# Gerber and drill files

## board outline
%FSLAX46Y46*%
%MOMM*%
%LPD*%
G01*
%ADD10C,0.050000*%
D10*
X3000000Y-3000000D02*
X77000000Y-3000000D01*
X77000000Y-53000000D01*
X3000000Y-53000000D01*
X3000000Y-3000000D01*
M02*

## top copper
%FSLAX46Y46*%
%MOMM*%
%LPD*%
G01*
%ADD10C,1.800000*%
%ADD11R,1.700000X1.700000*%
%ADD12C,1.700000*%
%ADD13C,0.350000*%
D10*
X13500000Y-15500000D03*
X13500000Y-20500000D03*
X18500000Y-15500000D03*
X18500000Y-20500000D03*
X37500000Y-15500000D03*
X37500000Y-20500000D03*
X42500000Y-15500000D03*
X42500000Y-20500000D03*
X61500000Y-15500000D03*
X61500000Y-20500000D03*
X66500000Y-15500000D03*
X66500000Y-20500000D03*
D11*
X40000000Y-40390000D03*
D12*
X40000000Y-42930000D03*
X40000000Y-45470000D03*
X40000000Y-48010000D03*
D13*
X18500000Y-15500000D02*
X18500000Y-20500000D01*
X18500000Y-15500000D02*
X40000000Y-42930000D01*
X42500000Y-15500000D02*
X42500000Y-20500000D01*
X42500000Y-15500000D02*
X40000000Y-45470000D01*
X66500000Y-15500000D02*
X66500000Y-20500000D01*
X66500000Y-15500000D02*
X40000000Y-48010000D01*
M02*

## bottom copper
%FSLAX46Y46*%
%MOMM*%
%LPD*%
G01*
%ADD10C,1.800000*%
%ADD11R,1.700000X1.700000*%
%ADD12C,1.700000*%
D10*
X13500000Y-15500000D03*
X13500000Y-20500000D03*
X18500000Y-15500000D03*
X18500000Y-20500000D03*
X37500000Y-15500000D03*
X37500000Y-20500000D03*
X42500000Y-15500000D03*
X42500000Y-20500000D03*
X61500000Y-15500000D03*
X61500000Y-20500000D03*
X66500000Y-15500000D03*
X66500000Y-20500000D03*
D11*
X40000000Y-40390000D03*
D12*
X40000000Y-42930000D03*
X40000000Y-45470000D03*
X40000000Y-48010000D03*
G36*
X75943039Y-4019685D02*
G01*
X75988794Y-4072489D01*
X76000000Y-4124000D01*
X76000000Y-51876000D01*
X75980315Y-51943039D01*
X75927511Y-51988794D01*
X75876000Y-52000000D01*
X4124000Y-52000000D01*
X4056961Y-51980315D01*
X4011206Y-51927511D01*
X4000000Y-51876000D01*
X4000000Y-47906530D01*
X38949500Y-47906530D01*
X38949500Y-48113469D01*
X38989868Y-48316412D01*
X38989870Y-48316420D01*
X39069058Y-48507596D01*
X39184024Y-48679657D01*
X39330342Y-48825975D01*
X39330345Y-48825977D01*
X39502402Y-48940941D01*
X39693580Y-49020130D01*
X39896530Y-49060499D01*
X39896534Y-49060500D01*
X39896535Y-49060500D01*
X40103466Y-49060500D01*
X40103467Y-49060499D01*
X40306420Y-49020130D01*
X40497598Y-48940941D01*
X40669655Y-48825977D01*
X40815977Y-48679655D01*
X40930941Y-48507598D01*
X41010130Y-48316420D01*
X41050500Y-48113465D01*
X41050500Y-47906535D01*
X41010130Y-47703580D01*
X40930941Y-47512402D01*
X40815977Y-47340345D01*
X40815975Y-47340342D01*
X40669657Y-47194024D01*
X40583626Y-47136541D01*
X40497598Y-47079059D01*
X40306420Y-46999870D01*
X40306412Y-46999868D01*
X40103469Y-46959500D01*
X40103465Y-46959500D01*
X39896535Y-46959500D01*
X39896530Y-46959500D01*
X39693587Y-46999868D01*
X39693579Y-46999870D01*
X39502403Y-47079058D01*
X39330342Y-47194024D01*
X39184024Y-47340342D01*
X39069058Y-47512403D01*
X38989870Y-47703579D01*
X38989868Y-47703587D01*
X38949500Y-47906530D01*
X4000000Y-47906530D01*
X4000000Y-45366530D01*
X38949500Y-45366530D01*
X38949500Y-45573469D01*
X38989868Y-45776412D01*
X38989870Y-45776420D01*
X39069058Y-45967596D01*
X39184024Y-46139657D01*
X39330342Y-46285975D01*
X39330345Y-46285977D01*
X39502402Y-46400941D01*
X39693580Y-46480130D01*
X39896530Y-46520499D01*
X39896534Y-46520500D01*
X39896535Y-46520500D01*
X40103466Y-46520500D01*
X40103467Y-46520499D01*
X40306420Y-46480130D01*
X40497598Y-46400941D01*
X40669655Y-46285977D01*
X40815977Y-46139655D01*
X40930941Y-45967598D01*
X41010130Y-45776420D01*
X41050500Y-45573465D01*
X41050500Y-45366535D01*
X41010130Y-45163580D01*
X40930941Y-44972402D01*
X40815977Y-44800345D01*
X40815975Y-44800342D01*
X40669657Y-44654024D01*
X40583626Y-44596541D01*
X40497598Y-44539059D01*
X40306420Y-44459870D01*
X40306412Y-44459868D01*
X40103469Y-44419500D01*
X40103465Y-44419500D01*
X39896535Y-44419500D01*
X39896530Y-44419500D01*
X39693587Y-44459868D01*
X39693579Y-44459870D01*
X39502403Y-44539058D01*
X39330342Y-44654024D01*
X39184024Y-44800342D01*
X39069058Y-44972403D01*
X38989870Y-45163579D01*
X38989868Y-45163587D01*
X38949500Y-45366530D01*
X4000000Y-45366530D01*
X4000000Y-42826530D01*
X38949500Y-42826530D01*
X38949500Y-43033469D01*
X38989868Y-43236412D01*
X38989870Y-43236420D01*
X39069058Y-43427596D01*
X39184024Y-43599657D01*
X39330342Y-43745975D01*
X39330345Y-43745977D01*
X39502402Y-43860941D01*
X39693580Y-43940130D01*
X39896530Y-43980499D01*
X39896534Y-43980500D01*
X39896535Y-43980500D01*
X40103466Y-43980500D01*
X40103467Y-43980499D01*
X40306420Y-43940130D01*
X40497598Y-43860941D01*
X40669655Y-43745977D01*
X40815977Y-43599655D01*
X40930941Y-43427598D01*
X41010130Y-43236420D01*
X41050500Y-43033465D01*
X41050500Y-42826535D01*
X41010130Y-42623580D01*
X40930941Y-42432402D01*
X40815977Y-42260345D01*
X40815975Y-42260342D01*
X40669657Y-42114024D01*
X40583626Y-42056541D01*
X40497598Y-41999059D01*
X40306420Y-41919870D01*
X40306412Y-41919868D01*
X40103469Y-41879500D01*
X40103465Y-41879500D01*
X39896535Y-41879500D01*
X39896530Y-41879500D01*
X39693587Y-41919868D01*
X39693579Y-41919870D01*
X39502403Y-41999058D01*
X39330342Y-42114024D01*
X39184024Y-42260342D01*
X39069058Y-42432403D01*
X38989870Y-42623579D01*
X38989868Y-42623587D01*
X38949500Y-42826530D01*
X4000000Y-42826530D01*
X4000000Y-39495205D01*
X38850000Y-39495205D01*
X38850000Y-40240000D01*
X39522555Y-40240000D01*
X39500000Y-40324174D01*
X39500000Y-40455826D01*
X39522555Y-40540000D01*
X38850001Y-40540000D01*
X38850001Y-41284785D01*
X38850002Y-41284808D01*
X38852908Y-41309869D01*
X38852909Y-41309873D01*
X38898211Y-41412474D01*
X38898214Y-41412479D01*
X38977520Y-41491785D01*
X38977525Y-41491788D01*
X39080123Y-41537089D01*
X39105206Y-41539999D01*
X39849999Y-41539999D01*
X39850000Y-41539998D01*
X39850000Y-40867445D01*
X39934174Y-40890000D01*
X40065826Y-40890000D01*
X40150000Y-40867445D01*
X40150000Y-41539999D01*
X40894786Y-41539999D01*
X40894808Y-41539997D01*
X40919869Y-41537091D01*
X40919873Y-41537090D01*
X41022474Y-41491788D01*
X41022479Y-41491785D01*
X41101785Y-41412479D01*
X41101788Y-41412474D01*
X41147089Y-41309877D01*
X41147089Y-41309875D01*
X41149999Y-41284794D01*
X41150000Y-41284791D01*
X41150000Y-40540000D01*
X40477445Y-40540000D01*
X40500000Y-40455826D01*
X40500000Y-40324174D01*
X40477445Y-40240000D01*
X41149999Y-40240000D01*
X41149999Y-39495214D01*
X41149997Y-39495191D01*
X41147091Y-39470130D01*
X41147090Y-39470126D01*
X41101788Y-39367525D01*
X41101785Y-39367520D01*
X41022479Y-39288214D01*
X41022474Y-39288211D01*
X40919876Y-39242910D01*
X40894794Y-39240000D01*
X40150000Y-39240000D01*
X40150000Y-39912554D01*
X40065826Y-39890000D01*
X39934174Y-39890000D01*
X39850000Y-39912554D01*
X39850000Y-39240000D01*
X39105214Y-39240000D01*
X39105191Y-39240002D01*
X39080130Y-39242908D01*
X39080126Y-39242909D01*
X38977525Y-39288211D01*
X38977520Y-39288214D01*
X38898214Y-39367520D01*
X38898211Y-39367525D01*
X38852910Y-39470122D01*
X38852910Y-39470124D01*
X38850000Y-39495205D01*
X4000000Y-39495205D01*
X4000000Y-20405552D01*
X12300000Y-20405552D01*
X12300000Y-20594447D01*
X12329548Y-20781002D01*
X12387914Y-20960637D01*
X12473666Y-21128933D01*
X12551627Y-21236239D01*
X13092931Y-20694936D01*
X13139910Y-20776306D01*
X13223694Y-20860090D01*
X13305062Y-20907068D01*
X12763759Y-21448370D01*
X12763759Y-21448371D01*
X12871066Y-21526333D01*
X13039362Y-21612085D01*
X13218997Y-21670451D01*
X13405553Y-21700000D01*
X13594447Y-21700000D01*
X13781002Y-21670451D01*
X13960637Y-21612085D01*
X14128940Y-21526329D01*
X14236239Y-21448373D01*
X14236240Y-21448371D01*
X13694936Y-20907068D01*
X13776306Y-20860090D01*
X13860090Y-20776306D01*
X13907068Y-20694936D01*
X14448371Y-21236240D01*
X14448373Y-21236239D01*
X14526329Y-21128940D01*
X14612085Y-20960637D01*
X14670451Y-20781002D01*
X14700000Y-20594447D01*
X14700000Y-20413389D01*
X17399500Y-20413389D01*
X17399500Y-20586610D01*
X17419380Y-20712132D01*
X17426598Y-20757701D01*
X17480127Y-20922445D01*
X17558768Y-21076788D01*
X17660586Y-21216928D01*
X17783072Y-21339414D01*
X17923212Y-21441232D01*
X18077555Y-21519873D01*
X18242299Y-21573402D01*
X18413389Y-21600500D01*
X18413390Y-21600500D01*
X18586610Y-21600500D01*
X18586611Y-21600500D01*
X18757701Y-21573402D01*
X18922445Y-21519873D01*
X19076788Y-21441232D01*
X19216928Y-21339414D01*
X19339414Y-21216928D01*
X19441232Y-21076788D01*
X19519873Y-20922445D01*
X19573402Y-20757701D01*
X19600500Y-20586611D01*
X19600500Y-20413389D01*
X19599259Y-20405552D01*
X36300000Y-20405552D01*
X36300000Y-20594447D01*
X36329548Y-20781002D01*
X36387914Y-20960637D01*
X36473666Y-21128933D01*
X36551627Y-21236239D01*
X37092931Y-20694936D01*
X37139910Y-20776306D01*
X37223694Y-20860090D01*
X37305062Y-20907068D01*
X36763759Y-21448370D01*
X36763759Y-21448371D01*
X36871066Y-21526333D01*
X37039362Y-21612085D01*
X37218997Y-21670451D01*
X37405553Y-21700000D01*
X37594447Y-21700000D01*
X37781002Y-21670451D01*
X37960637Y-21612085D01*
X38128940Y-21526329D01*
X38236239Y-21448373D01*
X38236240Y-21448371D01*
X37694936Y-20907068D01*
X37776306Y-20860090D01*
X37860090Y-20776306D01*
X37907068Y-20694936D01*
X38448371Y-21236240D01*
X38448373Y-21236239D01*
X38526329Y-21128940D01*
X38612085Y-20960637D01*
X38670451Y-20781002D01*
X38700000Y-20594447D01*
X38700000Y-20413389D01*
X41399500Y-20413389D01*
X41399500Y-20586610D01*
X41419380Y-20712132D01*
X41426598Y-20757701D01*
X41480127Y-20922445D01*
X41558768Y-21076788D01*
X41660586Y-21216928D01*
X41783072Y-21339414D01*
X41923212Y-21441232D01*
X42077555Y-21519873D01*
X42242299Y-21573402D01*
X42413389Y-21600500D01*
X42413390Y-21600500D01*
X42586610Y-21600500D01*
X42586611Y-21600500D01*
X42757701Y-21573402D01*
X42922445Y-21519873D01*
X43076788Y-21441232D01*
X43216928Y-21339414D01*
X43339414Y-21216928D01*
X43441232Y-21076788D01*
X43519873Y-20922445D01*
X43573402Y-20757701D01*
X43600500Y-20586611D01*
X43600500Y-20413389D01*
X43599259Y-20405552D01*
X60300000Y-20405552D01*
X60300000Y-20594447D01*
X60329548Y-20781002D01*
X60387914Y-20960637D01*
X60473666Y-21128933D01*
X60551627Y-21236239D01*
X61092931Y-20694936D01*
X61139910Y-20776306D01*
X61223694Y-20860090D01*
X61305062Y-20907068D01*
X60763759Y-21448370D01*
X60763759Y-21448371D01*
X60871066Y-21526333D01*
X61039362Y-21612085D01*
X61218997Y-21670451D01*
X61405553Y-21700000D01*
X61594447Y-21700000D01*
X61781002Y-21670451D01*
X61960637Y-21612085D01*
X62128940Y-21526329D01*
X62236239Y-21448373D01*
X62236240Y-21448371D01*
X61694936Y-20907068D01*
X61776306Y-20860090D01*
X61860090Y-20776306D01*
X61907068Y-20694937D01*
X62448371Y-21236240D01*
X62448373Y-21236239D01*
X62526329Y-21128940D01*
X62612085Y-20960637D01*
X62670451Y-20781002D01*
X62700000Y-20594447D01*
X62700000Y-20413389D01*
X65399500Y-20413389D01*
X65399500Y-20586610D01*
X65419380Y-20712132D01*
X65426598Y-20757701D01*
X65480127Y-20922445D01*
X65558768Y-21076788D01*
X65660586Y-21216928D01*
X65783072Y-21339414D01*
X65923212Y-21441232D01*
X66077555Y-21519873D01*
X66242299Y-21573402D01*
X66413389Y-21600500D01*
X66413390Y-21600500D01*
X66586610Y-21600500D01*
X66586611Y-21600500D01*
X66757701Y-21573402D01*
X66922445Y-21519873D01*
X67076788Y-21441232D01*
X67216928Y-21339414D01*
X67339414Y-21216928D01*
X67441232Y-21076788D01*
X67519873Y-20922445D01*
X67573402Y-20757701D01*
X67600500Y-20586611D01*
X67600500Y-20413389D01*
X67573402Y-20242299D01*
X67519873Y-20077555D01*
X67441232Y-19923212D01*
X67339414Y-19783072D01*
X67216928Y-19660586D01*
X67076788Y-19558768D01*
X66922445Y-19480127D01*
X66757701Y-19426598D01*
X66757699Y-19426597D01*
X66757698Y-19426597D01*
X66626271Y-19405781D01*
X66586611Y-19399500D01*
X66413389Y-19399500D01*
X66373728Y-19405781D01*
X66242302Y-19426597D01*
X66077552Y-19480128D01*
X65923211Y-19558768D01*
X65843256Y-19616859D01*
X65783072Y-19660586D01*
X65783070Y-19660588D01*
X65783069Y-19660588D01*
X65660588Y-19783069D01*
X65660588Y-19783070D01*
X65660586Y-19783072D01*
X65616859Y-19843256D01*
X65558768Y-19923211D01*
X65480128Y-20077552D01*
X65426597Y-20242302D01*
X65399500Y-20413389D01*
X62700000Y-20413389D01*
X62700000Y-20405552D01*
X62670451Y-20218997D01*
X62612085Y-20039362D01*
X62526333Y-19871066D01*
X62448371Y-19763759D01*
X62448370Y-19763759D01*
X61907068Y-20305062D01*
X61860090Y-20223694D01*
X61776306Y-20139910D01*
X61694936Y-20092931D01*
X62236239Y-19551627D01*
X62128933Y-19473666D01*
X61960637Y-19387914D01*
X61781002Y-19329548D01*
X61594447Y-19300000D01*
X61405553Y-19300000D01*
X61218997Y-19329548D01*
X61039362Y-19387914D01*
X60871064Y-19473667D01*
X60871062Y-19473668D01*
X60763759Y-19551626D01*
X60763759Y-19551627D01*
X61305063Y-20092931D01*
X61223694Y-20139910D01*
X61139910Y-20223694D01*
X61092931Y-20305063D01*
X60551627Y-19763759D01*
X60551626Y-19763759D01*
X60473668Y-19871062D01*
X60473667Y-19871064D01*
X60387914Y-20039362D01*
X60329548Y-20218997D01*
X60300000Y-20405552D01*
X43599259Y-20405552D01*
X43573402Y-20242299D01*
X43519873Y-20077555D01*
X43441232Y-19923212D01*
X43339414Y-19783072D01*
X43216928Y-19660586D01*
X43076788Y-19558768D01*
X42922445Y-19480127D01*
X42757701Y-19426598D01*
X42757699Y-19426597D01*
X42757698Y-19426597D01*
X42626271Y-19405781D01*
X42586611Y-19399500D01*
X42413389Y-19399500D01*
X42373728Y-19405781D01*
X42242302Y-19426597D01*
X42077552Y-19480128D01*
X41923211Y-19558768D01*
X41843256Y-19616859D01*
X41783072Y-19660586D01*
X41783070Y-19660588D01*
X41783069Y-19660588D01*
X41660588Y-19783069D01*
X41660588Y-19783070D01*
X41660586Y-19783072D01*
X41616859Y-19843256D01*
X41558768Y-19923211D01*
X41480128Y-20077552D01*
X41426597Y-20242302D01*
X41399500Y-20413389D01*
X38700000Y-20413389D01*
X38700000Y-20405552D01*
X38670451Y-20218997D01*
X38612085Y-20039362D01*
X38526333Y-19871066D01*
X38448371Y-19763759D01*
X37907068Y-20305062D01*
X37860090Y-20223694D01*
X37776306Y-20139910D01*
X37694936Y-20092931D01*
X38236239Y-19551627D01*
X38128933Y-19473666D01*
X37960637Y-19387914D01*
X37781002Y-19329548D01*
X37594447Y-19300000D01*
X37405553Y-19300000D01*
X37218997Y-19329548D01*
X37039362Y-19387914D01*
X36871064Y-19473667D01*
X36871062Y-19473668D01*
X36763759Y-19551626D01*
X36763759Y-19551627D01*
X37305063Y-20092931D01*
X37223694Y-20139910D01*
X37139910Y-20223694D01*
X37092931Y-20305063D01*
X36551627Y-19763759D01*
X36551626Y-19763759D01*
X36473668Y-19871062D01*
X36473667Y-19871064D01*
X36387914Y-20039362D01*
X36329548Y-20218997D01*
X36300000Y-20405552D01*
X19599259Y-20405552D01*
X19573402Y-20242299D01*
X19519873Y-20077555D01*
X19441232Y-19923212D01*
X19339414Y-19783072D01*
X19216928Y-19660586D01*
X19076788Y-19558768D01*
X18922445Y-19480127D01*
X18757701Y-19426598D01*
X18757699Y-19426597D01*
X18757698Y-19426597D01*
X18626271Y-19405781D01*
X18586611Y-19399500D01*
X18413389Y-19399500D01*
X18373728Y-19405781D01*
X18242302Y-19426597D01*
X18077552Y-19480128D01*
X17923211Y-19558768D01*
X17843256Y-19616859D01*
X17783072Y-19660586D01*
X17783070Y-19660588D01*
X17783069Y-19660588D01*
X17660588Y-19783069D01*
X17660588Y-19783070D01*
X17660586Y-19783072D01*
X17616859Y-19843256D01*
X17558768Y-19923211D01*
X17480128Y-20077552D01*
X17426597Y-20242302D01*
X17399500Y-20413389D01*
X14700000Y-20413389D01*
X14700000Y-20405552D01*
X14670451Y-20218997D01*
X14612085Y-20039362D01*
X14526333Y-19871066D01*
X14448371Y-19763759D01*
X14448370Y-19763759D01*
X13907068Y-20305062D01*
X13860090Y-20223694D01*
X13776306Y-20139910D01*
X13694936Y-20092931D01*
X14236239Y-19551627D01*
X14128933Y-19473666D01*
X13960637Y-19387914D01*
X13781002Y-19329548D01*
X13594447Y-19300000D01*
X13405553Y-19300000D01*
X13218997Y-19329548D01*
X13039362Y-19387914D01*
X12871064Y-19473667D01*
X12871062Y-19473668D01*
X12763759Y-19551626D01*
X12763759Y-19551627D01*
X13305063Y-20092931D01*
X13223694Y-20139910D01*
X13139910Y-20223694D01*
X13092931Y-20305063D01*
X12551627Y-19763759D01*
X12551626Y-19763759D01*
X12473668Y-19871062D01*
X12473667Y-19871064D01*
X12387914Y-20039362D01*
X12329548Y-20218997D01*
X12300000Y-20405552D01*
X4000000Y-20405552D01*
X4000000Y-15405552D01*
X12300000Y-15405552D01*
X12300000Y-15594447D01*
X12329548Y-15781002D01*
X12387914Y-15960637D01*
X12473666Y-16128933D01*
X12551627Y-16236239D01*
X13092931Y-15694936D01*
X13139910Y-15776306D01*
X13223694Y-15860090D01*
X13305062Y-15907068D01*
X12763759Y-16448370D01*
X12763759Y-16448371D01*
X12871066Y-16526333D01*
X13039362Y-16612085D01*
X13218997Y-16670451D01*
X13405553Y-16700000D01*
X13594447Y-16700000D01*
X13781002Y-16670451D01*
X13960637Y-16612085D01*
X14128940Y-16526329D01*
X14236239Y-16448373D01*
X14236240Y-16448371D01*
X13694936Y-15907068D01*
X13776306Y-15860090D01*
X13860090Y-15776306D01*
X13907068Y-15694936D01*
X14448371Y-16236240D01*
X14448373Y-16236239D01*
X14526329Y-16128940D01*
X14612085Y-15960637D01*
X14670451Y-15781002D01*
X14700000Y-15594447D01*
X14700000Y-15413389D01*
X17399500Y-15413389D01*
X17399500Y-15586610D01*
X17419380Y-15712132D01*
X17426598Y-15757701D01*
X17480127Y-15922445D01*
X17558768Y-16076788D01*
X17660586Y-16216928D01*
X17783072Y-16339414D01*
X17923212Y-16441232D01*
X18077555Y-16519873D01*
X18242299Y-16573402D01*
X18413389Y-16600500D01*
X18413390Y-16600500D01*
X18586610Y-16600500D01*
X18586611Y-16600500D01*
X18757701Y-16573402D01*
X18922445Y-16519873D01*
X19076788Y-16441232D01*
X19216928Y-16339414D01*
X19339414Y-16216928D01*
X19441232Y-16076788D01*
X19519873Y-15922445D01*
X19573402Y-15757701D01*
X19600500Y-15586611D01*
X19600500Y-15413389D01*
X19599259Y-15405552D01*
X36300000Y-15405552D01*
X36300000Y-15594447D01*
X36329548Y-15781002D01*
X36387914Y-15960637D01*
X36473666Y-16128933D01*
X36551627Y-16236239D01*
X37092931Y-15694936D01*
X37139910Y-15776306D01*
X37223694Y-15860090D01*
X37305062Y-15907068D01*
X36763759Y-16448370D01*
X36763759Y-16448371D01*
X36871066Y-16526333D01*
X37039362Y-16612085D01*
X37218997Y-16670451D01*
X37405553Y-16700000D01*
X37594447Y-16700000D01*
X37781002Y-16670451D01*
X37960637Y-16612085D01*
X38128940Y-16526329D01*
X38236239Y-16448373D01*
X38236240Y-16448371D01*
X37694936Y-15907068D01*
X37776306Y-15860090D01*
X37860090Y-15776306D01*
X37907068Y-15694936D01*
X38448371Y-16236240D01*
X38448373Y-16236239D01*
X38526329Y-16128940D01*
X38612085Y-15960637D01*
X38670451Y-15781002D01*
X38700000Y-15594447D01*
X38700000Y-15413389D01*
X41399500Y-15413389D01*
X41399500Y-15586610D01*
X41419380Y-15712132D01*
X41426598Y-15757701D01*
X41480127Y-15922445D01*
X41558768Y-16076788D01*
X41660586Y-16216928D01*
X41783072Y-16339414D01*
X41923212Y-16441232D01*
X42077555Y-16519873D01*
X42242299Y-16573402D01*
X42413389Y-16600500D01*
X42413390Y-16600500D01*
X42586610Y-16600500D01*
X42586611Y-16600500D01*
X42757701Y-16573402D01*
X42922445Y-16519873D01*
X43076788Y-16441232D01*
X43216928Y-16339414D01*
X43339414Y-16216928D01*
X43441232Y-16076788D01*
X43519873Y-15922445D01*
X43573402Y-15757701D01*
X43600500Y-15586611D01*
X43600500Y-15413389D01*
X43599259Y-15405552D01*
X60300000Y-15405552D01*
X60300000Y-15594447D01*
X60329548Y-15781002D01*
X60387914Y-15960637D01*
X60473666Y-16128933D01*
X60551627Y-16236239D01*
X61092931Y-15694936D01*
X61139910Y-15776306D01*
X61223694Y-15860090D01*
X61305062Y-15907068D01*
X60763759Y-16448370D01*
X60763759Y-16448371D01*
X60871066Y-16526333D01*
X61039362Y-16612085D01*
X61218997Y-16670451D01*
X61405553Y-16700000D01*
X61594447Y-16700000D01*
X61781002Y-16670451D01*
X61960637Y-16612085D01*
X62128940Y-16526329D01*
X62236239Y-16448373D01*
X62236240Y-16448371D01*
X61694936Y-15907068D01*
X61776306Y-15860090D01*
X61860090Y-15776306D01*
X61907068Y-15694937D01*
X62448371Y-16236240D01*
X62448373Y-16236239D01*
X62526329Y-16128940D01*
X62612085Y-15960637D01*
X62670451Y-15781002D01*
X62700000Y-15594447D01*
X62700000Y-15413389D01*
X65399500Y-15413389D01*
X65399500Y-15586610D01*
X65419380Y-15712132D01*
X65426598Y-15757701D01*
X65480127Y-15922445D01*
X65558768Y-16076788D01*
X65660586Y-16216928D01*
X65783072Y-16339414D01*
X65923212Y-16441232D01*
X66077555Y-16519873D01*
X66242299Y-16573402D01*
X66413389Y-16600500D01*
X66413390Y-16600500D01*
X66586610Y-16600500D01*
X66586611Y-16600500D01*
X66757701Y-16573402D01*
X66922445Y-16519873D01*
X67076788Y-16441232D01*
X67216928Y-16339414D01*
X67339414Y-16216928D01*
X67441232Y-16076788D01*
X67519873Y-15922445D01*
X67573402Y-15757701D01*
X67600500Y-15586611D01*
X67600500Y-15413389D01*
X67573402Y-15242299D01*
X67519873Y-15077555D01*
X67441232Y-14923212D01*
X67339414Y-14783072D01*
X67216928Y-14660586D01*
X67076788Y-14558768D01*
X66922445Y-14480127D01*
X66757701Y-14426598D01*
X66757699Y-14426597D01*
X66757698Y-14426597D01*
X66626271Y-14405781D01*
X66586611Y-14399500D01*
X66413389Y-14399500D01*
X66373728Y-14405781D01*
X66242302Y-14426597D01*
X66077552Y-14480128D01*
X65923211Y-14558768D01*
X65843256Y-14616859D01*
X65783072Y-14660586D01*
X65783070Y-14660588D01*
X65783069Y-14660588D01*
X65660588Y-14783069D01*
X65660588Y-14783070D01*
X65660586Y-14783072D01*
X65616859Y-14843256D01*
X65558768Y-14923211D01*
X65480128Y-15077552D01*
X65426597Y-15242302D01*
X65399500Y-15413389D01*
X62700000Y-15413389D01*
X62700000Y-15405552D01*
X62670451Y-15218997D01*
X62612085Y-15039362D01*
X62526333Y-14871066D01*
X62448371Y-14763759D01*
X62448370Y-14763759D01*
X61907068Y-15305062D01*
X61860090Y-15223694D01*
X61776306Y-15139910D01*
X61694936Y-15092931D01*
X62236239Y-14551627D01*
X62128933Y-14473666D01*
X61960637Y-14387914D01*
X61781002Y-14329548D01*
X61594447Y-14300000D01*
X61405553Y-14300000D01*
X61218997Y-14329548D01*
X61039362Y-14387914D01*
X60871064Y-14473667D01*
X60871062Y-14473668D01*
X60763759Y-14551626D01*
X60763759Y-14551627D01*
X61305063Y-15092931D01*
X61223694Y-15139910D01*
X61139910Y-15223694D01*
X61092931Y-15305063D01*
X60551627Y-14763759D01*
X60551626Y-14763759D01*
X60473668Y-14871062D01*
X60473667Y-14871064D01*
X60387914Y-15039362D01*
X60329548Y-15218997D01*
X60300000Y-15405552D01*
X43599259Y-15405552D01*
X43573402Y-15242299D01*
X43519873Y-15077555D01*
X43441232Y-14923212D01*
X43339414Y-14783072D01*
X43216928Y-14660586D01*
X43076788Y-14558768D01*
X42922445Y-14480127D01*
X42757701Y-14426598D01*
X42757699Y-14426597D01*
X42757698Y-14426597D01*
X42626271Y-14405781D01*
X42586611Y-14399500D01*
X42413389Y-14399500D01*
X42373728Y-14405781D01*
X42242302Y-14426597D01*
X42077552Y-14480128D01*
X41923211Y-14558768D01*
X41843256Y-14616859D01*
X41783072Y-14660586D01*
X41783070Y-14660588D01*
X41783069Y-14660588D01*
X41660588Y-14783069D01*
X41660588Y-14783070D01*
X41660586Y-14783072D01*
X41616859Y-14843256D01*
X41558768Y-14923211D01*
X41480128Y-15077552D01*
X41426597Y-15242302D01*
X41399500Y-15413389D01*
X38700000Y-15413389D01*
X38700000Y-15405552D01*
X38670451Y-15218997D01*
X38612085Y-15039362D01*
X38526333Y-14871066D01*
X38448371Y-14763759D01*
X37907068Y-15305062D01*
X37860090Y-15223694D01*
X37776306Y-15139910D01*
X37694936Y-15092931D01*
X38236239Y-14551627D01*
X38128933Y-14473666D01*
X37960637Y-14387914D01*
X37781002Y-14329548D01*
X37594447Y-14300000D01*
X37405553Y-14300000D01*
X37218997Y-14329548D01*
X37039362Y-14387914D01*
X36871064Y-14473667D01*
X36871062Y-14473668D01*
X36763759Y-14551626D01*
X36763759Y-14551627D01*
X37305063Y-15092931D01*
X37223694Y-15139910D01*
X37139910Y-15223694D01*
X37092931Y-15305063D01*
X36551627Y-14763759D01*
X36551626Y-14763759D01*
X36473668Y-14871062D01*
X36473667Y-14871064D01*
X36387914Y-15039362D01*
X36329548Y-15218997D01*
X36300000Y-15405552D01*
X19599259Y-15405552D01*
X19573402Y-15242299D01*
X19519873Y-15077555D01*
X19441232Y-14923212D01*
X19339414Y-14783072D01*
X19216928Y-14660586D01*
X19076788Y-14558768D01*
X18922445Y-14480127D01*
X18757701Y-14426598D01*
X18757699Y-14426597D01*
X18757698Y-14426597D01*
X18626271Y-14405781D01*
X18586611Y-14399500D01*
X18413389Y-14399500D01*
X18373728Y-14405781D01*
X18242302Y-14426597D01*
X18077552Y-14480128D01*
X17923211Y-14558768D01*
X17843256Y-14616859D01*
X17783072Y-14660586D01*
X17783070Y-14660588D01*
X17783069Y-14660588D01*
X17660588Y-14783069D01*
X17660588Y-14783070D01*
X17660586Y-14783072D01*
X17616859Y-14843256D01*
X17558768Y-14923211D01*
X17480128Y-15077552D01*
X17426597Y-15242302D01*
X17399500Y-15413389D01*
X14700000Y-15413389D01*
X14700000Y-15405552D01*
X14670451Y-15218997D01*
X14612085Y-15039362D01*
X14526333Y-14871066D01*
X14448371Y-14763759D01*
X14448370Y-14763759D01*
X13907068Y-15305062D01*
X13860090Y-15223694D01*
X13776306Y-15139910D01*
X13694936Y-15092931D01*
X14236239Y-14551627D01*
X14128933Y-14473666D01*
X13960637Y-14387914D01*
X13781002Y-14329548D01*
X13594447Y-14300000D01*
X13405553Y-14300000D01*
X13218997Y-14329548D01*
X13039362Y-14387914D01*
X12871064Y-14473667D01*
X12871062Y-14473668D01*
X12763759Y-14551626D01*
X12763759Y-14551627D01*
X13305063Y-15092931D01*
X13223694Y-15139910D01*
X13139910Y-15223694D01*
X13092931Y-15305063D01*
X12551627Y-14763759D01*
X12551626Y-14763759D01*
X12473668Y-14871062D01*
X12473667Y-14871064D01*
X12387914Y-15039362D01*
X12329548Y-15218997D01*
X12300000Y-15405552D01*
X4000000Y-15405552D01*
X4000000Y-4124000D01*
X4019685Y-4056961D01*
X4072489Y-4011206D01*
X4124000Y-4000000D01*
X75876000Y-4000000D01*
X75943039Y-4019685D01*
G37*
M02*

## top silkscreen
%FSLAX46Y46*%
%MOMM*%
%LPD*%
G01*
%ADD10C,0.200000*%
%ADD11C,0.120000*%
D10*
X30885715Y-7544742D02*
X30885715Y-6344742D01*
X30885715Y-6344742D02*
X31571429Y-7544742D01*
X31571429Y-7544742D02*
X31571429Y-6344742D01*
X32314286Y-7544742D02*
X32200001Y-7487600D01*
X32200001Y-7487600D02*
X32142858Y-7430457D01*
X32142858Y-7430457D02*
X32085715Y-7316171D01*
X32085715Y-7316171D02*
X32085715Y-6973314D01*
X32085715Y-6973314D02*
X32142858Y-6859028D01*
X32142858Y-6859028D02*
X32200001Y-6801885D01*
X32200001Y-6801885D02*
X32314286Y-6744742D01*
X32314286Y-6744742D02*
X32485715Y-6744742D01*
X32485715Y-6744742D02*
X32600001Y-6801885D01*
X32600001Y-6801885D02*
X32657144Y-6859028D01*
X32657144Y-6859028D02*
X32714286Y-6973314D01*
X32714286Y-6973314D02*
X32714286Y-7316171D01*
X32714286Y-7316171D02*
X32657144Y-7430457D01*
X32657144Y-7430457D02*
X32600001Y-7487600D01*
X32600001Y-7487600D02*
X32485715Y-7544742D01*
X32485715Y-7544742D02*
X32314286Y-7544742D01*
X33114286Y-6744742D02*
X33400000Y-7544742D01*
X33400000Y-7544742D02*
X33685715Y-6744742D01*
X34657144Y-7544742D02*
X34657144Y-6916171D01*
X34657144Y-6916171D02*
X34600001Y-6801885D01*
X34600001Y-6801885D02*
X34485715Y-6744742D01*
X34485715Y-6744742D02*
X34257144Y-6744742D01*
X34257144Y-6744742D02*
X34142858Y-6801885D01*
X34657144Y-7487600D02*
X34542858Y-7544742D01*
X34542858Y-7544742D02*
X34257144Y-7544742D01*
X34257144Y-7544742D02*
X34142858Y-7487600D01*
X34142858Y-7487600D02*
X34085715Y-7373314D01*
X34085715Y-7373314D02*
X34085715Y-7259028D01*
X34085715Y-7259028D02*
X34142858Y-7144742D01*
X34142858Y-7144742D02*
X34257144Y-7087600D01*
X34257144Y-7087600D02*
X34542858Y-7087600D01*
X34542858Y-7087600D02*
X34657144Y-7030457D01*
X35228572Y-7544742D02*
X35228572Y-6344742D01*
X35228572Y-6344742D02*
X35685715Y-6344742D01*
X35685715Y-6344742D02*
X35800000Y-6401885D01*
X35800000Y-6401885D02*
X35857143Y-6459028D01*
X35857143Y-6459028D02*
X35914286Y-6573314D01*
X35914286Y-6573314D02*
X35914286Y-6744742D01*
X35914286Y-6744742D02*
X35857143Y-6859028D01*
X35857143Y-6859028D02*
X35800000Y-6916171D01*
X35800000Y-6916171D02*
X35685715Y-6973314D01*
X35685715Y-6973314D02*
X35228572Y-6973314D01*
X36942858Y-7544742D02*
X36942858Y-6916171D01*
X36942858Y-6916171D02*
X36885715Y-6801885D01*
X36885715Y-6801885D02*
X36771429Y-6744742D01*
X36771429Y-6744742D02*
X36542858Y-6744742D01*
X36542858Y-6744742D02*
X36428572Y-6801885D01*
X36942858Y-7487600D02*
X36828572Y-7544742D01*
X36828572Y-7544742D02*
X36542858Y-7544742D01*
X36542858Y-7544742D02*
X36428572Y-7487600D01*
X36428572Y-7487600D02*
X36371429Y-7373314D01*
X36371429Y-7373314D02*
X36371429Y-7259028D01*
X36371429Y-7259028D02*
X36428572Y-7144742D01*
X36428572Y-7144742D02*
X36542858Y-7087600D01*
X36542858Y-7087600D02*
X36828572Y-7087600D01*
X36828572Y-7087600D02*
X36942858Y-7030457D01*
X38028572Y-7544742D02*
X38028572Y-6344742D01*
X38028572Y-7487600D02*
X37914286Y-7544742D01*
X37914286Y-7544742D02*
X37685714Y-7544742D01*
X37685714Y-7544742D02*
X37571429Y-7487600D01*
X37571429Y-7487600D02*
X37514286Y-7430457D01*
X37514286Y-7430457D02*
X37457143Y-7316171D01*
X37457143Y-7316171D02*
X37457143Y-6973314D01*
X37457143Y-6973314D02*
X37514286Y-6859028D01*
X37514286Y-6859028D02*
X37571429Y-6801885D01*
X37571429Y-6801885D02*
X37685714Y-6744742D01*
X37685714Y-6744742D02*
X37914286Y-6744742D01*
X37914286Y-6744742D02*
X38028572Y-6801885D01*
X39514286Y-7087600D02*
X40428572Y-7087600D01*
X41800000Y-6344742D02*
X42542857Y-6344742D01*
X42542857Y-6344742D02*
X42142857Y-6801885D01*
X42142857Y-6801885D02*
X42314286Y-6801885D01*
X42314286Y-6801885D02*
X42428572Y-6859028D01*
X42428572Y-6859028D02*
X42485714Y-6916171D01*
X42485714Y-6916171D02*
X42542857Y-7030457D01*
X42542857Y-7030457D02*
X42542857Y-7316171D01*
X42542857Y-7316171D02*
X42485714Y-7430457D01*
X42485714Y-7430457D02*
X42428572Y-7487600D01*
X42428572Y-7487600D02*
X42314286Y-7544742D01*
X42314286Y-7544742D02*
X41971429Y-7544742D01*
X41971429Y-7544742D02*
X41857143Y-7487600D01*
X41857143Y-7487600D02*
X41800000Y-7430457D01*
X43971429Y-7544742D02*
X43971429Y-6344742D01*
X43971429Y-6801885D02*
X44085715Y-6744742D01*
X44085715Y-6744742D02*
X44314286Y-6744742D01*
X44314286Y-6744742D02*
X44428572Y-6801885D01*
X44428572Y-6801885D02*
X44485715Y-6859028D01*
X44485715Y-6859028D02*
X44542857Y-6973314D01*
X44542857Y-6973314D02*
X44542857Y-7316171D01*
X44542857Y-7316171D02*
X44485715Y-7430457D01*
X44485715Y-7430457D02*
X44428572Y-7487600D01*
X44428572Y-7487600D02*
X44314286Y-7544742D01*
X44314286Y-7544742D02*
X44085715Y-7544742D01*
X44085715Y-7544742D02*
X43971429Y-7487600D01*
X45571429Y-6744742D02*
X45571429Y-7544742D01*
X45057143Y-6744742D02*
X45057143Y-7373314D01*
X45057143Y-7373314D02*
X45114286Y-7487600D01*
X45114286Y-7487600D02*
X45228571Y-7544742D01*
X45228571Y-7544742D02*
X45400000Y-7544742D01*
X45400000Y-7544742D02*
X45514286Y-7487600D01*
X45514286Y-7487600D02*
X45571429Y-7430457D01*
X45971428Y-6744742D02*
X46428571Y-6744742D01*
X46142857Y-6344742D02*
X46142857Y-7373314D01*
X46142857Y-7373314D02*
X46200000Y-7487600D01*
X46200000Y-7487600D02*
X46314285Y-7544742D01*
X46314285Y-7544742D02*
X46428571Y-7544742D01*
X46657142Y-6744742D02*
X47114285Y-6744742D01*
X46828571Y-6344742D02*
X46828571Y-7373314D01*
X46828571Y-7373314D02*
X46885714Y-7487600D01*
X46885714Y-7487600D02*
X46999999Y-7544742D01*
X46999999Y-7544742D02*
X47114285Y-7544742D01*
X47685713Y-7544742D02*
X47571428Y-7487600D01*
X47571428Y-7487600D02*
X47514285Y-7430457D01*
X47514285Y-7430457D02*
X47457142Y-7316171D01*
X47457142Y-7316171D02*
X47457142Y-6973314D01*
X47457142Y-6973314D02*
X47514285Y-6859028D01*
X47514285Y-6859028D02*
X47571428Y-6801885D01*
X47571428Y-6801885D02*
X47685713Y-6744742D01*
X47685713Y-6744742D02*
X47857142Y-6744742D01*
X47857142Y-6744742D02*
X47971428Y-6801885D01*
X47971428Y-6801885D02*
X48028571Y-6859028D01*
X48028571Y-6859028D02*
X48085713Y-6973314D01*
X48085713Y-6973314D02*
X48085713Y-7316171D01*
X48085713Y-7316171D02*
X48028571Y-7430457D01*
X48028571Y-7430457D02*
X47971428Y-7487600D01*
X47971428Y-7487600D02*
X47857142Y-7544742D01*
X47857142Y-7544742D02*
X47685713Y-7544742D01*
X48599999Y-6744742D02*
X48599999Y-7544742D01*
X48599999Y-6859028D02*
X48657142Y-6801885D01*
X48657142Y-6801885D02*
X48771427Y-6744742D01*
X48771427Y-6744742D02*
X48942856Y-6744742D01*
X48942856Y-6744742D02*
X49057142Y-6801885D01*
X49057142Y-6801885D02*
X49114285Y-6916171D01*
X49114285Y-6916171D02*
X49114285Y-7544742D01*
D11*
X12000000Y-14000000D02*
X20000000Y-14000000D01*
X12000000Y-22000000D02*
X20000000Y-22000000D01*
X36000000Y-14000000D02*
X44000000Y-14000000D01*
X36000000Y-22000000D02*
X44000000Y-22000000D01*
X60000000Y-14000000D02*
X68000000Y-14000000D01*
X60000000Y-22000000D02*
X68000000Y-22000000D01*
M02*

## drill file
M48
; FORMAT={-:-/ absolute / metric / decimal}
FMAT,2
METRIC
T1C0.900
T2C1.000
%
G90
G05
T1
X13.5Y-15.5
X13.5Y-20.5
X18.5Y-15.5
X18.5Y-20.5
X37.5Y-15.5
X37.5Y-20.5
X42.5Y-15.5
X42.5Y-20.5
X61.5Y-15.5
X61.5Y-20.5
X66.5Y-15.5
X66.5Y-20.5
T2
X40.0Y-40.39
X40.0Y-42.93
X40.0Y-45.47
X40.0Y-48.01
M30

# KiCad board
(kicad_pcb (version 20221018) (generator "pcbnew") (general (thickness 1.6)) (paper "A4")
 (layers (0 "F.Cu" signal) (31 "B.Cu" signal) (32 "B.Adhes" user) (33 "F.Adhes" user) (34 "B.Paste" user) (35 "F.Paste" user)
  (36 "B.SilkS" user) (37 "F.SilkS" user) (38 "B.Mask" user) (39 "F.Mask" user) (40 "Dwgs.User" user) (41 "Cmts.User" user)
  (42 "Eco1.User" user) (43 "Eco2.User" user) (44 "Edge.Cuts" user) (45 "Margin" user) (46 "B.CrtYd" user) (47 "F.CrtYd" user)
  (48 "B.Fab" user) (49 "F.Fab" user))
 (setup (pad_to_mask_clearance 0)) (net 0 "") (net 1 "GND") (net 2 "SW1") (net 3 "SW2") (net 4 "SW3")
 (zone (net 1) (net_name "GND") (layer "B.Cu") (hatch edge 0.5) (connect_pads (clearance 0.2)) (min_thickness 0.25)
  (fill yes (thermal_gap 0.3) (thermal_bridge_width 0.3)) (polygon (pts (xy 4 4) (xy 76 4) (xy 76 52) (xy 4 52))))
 (gr_rect (start 3 3) (end 77 53) (stroke (width 0.05) (type default)) (fill none) (layer "Edge.Cuts"))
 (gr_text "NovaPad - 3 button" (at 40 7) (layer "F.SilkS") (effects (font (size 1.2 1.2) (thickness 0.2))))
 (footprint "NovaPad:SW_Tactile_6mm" (layer "F.Cu") (at 16 18)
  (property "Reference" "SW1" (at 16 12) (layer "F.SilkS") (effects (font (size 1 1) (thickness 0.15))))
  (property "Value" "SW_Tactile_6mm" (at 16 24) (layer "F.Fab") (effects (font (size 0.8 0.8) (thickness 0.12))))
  (fp_line (start -4 -4) (end 4 -4) (stroke (width 0.12) (type default)) (layer "F.SilkS"))
  (fp_line (start -4 4) (end 4 4) (stroke (width 0.12) (type default)) (layer "F.SilkS"))
  (pad "1" thru_hole circle (at -2.5 -2.5) (size 1.8 1.8) (drill 0.9) (layers "*.Cu" "*.Mask") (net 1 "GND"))
  (pad "1" thru_hole circle (at -2.5 2.5) (size 1.8 1.8) (drill 0.9) (layers "*.Cu" "*.Mask") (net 1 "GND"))
  (pad "2" thru_hole circle (at 2.5 -2.5) (size 1.8 1.8) (drill 0.9) (layers "*.Cu" "*.Mask") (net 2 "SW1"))
  (pad "2" thru_hole circle (at 2.5 2.5) (size 1.8 1.8) (drill 0.9) (layers "*.Cu" "*.Mask") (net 2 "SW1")))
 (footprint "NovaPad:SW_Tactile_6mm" (layer "F.Cu") (at 40 18)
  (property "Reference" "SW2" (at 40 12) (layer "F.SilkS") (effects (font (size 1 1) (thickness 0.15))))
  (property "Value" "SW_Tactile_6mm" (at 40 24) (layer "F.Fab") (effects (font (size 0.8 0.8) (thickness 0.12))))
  (fp_line (start -4 -4) (end 4 -4) (stroke (width 0.12) (type default)) (layer "F.SilkS"))
  (fp_line (start -4 4) (end 4 4) (stroke (width 0.12) (type default)) (layer "F.SilkS"))
  (pad "1" thru_hole circle (at -2.5 -2.5) (size 1.8 1.8) (drill 0.9) (layers "*.Cu" "*.Mask") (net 1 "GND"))
  (pad "1" thru_hole circle (at -2.5 2.5) (size 1.8 1.8) (drill 0.9) (layers "*.Cu" "*.Mask") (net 1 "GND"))
  (pad "2" thru_hole circle (at 2.5 -2.5) (size 1.8 1.8) (drill 0.9) (layers "*.Cu" "*.Mask") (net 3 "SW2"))
  (pad "2" thru_hole circle (at 2.5 2.5) (size 1.8 1.8) (drill 0.9) (layers "*.Cu" "*.Mask") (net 3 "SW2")))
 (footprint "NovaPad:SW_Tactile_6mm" (layer "F.Cu") (at 64 18)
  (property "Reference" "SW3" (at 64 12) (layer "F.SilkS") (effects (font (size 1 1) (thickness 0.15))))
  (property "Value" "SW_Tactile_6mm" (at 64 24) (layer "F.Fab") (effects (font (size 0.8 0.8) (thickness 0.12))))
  (fp_line (start -4 -4) (end 4 -4) (stroke (width 0.12) (type default)) (layer "F.SilkS"))
  (fp_line (start -4 4) (end 4 4) (stroke (width 0.12) (type default)) (layer "F.SilkS"))
  (pad "1" thru_hole circle (at -2.5 -2.5) (size 1.8 1.8) (drill 0.9) (layers "*.Cu" "*.Mask") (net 1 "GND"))
  (pad "1" thru_hole circle (at -2.5 2.5) (size 1.8 1.8) (drill 0.9) (layers "*.Cu" "*.Mask") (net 1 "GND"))
  (pad "2" thru_hole circle (at 2.5 -2.5) (size 1.8 1.8) (drill 0.9) (layers "*.Cu" "*.Mask") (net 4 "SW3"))
  (pad "2" thru_hole circle (at 2.5 2.5) (size 1.8 1.8) (drill 0.9) (layers "*.Cu" "*.Mask") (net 4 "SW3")))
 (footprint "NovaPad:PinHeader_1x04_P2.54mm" (layer "F.Cu") (at 40 44.2)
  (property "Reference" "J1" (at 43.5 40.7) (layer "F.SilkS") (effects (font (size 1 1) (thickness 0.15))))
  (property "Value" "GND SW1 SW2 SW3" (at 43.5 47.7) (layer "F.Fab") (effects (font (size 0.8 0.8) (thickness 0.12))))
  (pad "1" thru_hole rect (at 0 -3.81) (size 1.7 1.7) (drill 1) (layers "*.Cu" "*.Mask") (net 1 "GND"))
  (pad "2" thru_hole circle (at 0 -1.27) (size 1.7 1.7) (drill 1) (layers "*.Cu" "*.Mask") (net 2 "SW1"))
  (pad "3" thru_hole circle (at 0 1.27) (size 1.7 1.7) (drill 1) (layers "*.Cu" "*.Mask") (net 3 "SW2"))
  (pad "4" thru_hole circle (at 0 3.81) (size 1.7 1.7) (drill 1) (layers "*.Cu" "*.Mask") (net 4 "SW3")))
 (segment (start 18.5 15.5) (end 18.5 20.5) (width 0.35) (layer "F.Cu") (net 2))
 (segment (start 18.5 15.5) (end 40 42.93) (width 0.35) (layer "F.Cu") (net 2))
 (segment (start 42.5 15.5) (end 42.5 20.5) (width 0.35) (layer "F.Cu") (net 3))
 (segment (start 42.5 15.5) (end 40 45.47) (width 0.35) (layer "F.Cu") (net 3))
 (segment (start 66.5 15.5) (end 66.5 20.5) (width 0.35) (layer "F.Cu") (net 4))
 (segment (start 66.5 15.5) (end 40 48.01) (width 0.35) (layer "F.Cu") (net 4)))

